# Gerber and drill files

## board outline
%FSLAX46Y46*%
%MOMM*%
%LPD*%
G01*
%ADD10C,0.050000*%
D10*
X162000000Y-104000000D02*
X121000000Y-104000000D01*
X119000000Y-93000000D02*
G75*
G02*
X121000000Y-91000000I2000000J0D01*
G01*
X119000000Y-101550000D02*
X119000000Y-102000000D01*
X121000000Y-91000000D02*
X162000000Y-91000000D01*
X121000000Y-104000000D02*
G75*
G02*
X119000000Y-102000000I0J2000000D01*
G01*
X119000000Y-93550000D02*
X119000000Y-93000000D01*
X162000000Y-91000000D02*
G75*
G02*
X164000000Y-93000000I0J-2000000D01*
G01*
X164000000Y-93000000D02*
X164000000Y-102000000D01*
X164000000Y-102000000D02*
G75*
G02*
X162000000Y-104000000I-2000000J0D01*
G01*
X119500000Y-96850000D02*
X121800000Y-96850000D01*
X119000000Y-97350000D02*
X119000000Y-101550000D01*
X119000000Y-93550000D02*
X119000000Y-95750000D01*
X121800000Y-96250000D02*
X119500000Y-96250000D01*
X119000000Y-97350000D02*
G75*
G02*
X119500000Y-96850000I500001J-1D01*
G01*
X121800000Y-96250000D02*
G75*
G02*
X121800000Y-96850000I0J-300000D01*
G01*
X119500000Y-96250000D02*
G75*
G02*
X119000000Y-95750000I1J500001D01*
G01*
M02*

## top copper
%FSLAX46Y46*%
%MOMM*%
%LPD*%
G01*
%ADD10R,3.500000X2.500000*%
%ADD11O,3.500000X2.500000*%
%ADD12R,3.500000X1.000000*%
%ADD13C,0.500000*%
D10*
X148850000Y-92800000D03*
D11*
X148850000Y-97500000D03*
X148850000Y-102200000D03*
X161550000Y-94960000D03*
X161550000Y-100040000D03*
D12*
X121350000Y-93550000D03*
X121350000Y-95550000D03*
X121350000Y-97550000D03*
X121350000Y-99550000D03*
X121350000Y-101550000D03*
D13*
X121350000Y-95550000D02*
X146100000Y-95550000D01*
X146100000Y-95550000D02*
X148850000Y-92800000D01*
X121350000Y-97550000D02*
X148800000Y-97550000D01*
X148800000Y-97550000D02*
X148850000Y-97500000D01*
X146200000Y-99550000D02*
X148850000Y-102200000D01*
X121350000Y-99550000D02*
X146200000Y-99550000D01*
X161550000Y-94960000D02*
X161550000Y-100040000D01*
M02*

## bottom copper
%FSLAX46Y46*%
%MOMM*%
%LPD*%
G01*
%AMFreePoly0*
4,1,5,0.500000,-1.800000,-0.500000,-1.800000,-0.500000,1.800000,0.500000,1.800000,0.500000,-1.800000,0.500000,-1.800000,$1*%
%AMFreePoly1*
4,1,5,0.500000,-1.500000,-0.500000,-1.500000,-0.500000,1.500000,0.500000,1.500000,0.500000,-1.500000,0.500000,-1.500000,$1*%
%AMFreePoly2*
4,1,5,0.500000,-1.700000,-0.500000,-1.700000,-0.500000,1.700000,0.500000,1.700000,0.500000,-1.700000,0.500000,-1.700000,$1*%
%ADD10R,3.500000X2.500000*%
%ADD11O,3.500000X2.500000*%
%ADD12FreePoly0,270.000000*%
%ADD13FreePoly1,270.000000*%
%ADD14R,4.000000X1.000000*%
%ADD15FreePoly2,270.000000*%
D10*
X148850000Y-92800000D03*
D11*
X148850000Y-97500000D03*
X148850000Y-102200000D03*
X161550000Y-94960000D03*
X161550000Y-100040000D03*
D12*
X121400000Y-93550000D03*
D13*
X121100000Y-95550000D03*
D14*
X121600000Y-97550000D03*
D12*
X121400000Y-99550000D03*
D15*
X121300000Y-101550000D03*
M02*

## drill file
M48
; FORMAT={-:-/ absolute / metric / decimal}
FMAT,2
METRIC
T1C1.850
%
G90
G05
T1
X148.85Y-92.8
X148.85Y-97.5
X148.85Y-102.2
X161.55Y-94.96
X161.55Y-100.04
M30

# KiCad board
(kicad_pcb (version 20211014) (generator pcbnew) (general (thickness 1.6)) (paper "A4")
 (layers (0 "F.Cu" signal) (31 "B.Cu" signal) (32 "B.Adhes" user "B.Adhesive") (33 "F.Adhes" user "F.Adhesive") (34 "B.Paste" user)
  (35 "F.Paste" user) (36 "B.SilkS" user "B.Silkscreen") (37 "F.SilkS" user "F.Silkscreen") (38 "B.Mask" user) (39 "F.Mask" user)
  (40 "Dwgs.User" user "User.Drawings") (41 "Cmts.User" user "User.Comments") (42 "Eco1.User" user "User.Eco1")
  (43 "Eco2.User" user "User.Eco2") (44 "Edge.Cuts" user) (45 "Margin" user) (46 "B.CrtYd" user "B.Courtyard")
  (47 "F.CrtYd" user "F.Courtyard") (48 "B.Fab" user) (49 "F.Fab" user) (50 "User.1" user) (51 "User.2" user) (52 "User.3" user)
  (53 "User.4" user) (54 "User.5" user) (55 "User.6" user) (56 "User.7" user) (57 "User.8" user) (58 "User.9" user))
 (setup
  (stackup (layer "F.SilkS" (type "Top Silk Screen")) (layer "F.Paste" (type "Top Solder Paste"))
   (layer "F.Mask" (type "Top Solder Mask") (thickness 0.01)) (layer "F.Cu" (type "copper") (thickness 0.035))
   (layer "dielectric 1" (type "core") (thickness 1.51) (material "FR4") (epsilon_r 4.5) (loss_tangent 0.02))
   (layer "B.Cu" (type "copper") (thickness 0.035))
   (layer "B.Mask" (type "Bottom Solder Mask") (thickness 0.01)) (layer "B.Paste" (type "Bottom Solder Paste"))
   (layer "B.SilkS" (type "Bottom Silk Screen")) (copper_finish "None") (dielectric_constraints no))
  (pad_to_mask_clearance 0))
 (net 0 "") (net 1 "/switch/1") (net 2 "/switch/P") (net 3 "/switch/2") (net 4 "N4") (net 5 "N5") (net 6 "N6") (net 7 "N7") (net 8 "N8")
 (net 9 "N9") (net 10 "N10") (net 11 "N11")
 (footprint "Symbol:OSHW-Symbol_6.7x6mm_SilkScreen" (layer "F.Cu") (at 137 100)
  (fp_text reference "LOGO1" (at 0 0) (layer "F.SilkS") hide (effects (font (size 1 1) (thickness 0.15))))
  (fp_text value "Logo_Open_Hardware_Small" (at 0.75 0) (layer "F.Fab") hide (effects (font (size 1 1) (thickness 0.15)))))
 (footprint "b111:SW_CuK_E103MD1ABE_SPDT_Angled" (layer "F.Cu") (at 148.85 97.5 90)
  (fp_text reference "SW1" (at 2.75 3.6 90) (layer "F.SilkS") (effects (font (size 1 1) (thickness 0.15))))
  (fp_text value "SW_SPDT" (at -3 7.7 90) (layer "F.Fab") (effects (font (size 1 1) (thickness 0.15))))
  (pad "1" thru_hole rect (at 4.7 0 90) (size 2.5 3.5) (drill 1.85) (layers *.Cu *.Mask) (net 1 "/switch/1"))
  (pad "2" thru_hole oval (at 0 0 90) (size 2.5 3.5) (drill 1.85) (layers *.Cu *.Mask) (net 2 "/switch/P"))
  (pad "3" thru_hole oval (at -4.7 0 270) (size 2.5 3.5) (drill 1.85) (layers *.Cu *.Mask) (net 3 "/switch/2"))
  (pad "S1" thru_hole oval (at 2.54 12.7 90) (size 2.5 3.5) (drill 1.85) (layers *.Cu *.Mask) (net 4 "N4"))
  (pad "S2" thru_hole oval (at -2.54 12.7 90) (size 2.5 3.5) (drill 1.85) (layers *.Cu *.Mask) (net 4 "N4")))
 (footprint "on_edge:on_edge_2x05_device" (layer "F.Cu") (at 119 97.55 -90)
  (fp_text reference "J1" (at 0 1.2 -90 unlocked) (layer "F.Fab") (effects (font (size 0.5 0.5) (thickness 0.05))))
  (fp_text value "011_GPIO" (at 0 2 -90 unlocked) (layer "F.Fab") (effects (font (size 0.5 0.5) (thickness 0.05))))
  (fp_line (start -0.7 -0.5) (end -0.7 -2.8) (layer "Edge.Cuts") (width 0.05))
  (fp_line (start -0.2 0) (end 4 0) (layer "Edge.Cuts") (width 0.05))
  (fp_line (start -4 0) (end -1.8 0) (layer "Edge.Cuts") (width 0.05))
  (fp_line (start -1.3 -2.8) (end -1.3 -0.5) (layer "Edge.Cuts") (width 0.05))
  (fp_arc (start -0.2 0) (mid -0.553553 -0.146447) (end -0.7 -0.5) (layer "Edge.Cuts") (width 0.05))
  (fp_arc (start -1.3 -2.8) (mid -1 -3.1) (end -0.7 -2.8) (layer "Edge.Cuts") (width 0.05))
  (fp_arc (start -1.3 -0.5) (mid -1.446447 -0.146447) (end -1.8 0) (layer "Edge.Cuts") (width 0.05))
  (pad "1" smd rect (at -4 -2.35 90) (size 1 3.5) (layers "F.Cu" "F.Mask") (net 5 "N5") (zone_connect 0))
  (pad "2" smd rect (at -2 -2.35 270) (size 1 3.5) (layers "F.Cu" "F.Mask") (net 1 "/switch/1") (zone_connect 0))
  (pad "3" smd rect (at 0 -2.35 270) (size 1 3.5) (layers "F.Cu" "F.Mask") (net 2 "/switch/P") (zone_connect 0))
  (pad "4" smd rect (at 2 -2.35 90) (size 1 3.5) (layers "F.Cu" "F.Mask") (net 3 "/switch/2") (zone_connect 0))
  (pad "5" smd rect (at 4 -2.35 90) (size 1 3.5) (layers "F.Cu" "F.Mask") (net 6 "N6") (zone_connect 0))
  (pad "6" smd custom (at -4 -2.4 270) (size 1 3.6) (layers "B.Cu" "B.Mask") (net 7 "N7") (zone_connect 0)
   (options (clearance outline) (anchor rect)) (primitives))
  (pad "7" smd custom (at -2 -2.1 270) (size 1 3) (layers "B.Cu" "B.Mask") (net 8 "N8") (zone_connect 0)
   (options (clearance outline) (anchor rect)) (primitives))
  (pad "8" smd rect (at 0 -2.6 270) (size 1 4) (layers "B.Cu" "B.Mask") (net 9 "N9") (zone_connect 0))
  (pad "9" smd custom (at 2 -2.4 270) (size 1 3.6) (layers "B.Cu" "B.Mask") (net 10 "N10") (zone_connect 0)
   (options (clearance outline) (anchor rect)) (primitives))
  (pad "10" smd custom (at 4 -2.3 270) (size 1 3.4) (layers "B.Cu" "B.Mask") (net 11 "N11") (zone_connect 0)
   (options (clearance outline) (anchor rect)) (primitives))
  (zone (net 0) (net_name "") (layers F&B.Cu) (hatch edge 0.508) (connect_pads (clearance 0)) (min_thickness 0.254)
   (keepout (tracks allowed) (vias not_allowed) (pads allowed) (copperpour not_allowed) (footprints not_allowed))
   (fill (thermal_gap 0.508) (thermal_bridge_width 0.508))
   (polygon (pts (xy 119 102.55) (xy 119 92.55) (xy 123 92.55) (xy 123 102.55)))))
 (gr_line (start 162 104) (end 121 104) (layer "Edge.Cuts") (width 0.05))
 (gr_arc (start 119 93) (mid 119.585786 91.585786) (end 121 91) (layer "Edge.Cuts") (width 0.05))
 (gr_line (start 119 101.55) (end 119 102) (layer "Edge.Cuts") (width 0.05))
 (gr_line (start 121 91) (end 162 91) (layer "Edge.Cuts") (width 0.05))
 (gr_arc (start 121 104) (mid 119.585786 103.414214) (end 119 102) (layer "Edge.Cuts") (width 0.05))
 (gr_line (start 119 93.55) (end 119 93) (layer "Edge.Cuts") (width 0.05))
 (gr_arc (start 162 91) (mid 163.414214 91.585786) (end 164 93) (layer "Edge.Cuts") (width 0.05))
 (gr_line (start 164 93) (end 164 102) (layer "Edge.Cuts") (width 0.05))
 (gr_arc (start 164 102) (mid 163.414214 103.414214) (end 162 104) (layer "Edge.Cuts") (width 0.05))
 (segment (start 121.35 95.55) (end 146.1 95.55) (width 0.5) (layer "F.Cu") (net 1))
 (segment (start 146.1 95.55) (end 148.85 92.8) (width 0.5) (layer "F.Cu") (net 1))
 (segment (start 121.35 97.55) (end 148.8 97.55) (width 0.5) (layer "F.Cu") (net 2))
 (segment (start 148.8 97.55) (end 148.85 97.5) (width 0.5) (layer "F.Cu") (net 2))
 (segment (start 146.2 99.55) (end 148.85 102.2) (width 0.5) (layer "F.Cu") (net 3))
 (segment (start 121.35 99.55) (end 146.2 99.55) (width 0.5) (layer "F.Cu") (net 3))
 (segment (start 161.55 94.96) (end 161.55 100.04) (width 0.5) (layer "F.Cu") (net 4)))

